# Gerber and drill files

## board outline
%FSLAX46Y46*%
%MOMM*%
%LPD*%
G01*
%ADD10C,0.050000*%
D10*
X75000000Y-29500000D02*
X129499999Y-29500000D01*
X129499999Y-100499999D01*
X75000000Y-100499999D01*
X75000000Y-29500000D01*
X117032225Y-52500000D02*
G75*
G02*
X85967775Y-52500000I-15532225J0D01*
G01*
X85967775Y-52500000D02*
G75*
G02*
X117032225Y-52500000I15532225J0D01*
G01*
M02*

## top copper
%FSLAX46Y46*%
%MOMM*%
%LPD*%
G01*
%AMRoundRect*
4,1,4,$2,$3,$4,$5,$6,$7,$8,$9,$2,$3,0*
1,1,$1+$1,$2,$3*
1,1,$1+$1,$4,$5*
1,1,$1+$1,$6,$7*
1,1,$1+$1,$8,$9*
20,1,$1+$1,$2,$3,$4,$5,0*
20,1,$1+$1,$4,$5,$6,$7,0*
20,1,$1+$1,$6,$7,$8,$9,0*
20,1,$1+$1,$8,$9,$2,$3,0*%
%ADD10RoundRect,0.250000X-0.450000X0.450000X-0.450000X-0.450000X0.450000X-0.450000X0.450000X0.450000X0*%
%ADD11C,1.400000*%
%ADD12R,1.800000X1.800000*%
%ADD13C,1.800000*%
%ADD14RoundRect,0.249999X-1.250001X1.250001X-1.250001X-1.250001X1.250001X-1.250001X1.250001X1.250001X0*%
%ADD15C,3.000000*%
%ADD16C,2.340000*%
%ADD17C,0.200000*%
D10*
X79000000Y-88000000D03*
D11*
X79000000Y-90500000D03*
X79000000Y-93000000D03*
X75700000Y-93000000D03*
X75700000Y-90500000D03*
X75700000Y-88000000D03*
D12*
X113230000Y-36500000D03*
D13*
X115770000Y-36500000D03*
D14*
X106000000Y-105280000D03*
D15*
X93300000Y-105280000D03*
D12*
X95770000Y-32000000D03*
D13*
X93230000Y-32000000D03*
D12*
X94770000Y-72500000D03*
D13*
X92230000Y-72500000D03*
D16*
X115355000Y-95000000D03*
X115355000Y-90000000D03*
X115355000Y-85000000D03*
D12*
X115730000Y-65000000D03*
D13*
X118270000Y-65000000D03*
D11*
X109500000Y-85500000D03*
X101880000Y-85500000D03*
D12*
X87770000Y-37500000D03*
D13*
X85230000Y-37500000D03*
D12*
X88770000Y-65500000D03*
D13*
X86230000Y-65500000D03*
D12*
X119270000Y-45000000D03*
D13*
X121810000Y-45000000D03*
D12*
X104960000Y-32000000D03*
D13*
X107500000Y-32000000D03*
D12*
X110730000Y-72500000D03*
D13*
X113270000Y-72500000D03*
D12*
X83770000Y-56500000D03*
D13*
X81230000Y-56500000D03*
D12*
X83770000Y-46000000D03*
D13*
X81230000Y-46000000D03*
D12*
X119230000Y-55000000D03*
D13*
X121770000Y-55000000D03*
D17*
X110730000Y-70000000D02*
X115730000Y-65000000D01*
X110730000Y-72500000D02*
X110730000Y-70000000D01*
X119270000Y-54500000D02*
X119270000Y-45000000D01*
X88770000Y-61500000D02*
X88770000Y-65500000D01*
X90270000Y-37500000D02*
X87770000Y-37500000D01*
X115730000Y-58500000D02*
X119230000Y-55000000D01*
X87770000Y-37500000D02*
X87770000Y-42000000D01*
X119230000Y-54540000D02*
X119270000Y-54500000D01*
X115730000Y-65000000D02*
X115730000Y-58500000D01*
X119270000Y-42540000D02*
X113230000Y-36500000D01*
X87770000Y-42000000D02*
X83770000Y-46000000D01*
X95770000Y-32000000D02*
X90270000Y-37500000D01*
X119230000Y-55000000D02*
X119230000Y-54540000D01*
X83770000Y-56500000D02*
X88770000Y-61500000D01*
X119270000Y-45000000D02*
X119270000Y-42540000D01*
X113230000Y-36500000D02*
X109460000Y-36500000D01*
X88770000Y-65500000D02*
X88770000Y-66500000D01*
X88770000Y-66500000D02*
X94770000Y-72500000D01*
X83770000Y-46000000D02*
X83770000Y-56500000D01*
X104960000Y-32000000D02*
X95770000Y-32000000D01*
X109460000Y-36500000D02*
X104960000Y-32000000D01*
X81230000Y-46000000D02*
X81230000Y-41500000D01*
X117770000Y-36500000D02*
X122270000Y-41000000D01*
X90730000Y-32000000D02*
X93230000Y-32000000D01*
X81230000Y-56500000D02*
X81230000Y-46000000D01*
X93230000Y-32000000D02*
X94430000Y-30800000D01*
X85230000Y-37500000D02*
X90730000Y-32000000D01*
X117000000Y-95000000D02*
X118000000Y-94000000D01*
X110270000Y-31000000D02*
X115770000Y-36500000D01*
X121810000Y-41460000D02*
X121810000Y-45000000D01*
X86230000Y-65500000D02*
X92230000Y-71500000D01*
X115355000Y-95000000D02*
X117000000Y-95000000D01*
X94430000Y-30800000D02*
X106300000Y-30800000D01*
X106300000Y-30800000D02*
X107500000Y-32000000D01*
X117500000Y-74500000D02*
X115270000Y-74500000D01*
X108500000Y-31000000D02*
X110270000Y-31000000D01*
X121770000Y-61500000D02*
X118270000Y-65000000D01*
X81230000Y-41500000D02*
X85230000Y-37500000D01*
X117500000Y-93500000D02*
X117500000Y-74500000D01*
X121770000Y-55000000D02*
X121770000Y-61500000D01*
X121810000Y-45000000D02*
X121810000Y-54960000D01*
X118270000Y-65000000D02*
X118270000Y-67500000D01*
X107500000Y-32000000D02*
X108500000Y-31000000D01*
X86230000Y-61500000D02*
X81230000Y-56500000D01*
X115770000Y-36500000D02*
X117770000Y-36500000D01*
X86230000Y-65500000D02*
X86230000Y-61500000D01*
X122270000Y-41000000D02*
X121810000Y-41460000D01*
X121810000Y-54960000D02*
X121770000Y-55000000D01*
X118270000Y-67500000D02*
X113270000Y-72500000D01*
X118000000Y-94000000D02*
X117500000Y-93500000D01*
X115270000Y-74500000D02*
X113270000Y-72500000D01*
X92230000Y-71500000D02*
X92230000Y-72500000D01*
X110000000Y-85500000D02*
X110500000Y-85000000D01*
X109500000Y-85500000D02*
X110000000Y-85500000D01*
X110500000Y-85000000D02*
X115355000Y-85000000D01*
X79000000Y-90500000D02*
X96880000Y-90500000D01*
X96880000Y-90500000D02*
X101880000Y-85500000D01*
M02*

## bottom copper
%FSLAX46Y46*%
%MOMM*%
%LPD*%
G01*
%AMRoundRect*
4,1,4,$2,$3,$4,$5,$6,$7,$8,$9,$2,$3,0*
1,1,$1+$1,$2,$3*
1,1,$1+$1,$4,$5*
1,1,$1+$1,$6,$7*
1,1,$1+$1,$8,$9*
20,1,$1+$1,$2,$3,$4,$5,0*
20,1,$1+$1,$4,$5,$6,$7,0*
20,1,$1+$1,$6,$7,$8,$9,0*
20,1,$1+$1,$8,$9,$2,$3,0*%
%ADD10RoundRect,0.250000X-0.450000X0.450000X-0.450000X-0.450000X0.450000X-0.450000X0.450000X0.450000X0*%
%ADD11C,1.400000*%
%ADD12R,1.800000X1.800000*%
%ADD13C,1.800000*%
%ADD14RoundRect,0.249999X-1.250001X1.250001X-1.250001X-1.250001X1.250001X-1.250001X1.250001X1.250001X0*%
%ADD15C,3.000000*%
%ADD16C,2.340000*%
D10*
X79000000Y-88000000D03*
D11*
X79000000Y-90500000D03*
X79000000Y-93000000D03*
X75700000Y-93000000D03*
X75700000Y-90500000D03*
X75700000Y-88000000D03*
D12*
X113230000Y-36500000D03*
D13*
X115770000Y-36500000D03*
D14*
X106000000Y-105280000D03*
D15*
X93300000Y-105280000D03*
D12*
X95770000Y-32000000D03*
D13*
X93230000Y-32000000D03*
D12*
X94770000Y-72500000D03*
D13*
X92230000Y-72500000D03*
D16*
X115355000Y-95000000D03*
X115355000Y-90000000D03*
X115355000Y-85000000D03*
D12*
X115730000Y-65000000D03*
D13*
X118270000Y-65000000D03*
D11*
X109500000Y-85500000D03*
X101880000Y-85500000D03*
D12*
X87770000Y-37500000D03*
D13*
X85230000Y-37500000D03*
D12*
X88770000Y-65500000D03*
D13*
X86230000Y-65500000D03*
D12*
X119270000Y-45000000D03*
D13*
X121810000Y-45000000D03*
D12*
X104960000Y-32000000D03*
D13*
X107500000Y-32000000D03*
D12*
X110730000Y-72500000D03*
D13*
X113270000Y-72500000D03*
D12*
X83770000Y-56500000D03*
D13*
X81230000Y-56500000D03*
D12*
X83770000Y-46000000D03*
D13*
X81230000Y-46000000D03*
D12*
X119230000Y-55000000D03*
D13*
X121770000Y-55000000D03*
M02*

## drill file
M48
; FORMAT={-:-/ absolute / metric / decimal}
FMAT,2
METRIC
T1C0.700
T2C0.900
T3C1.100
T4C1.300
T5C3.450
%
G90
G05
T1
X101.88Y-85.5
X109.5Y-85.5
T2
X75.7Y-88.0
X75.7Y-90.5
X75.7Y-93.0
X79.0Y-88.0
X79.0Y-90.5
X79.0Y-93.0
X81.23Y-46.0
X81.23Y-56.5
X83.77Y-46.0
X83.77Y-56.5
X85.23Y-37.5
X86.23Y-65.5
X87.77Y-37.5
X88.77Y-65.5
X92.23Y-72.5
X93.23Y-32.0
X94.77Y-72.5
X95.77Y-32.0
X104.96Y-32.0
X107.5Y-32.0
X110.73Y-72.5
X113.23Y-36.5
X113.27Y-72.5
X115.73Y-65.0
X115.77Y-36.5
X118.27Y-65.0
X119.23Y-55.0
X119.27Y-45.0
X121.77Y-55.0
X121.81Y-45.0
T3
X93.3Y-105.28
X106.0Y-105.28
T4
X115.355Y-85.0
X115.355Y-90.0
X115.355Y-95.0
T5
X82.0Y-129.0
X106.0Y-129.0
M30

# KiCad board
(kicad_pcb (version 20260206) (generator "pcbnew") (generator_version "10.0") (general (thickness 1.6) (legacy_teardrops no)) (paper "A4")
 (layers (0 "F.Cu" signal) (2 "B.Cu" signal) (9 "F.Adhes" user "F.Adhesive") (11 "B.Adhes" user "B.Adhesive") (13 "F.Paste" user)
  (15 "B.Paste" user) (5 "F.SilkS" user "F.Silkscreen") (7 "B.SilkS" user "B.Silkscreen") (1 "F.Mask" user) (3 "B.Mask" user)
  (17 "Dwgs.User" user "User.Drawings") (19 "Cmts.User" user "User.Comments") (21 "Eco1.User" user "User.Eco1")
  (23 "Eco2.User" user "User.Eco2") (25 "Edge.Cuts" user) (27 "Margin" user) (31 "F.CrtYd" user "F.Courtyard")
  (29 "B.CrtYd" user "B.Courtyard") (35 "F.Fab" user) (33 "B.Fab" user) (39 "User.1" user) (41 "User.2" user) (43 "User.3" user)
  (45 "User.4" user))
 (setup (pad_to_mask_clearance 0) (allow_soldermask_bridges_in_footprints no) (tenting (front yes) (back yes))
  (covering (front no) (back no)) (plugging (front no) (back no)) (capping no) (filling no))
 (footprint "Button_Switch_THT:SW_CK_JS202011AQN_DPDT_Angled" (layer "F.Cu") (at 79 88 -90)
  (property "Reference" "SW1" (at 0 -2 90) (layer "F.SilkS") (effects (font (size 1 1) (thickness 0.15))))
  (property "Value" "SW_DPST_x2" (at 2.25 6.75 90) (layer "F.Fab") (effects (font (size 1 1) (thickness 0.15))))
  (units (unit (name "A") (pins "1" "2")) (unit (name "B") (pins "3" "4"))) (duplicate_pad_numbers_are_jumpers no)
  (pad "1" thru_hole roundrect (at 0 0 270) (size 1.4 1.4) (drill 0.9) (layers "*.Cu" "*.Mask") (remove_unused_layers no)
   (roundrect_rratio 0.1785714286) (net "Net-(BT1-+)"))
  (pad "2" thru_hole circle (at 2.5 0 270) (size 1.4 1.4) (drill 0.9) (layers "*.Cu" "*.Mask") (remove_unused_layers no)
   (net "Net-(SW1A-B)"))
  (pad "3" thru_hole circle (at 5 0 270) (size 1.4 1.4) (drill 0.9) (layers "*.Cu" "*.Mask") (remove_unused_layers no))
  (pad "4" thru_hole circle (at 5 3.3 270) (size 1.4 1.4) (drill 0.9) (layers "*.Cu" "*.Mask") (remove_unused_layers no))
  (pad "5" thru_hole circle (at 2.5 3.3 270) (size 1.4 1.4) (drill 0.9) (layers "*.Cu" "*.Mask") (remove_unused_layers no))
  (pad "6" thru_hole circle (at 0 3.3 270) (size 1.4 1.4) (drill 0.9) (layers "*.Cu" "*.Mask") (remove_unused_layers no)))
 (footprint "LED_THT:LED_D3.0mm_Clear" (layer "F.Cu") (at 113.23 36.5)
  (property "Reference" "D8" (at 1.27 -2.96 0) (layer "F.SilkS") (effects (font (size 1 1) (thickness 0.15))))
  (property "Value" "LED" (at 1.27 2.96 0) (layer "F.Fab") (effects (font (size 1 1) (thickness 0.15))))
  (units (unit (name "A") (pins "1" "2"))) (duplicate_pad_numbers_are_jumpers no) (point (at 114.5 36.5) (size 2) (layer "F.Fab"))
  (pad "1" thru_hole rect (at 0 0) (size 1.8 1.8) (drill 0.9) (layers "*.Cu" "*.Mask") (remove_unused_layers no) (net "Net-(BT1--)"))
  (pad "2" thru_hole circle (at 2.54 0) (size 1.8 1.8) (drill 0.9) (layers "*.Cu" "*.Mask") (remove_unused_layers no) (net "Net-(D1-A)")))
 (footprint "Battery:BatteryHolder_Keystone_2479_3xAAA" (layer "F.Cu") (at 106 105.28 -90)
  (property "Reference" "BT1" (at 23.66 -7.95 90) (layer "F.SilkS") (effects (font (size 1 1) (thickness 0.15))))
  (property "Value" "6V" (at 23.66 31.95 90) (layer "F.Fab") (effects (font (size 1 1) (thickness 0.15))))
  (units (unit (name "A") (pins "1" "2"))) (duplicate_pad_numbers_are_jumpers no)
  (pad "" np_thru_hole circle (at 23.72 0 270) (size 3.45 3.45) (drill 3.45) (layers "*.Cu" "*.Mask"))
  (pad "" np_thru_hole circle (at 23.72 24 270) (size 3.45 3.45) (drill 3.45) (layers "*.Cu" "*.Mask"))
  (pad "1" thru_hole roundrect (at 0 0 270) (size 3 3) (drill 1.1) (layers "*.Cu" "*.Mask") (remove_unused_layers no)
   (roundrect_rratio 0.083333) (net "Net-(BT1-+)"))
  (pad "2" thru_hole circle (at 0 12.7 270) (size 3 3) (drill 1.1) (layers "*.Cu" "*.Mask") (remove_unused_layers no) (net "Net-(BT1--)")))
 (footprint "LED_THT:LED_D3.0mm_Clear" (layer "F.Cu") (at 95.77 32 180)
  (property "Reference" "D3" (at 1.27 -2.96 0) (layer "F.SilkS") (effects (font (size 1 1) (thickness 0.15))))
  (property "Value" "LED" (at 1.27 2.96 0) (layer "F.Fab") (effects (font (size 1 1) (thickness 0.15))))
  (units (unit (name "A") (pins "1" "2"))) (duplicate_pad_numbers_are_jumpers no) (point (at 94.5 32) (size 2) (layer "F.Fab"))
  (pad "1" thru_hole rect (at 0 0 180) (size 1.8 1.8) (drill 0.9) (layers "*.Cu" "*.Mask") (remove_unused_layers no) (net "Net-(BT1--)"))
  (pad "2" thru_hole circle (at 2.54 0 180) (size 1.8 1.8) (drill 0.9) (layers "*.Cu" "*.Mask") (remove_unused_layers no) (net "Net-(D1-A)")))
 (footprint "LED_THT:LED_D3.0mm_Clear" (layer "F.Cu") (at 94.77 72.5 180)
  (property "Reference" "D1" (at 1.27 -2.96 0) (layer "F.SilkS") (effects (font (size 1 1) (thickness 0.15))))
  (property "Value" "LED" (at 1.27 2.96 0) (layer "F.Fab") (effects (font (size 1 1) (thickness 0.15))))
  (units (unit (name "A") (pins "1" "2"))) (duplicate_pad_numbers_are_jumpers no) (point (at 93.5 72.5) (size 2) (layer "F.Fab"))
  (pad "1" thru_hole rect (at 0 0 180) (size 1.8 1.8) (drill 0.9) (layers "*.Cu" "*.Mask") (remove_unused_layers no) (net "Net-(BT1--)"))
  (pad "2" thru_hole circle (at 2.54 0 180) (size 1.8 1.8) (drill 0.9) (layers "*.Cu" "*.Mask") (remove_unused_layers no) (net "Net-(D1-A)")))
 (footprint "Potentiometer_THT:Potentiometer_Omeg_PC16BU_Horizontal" (layer "F.Cu") (at 115.355 95)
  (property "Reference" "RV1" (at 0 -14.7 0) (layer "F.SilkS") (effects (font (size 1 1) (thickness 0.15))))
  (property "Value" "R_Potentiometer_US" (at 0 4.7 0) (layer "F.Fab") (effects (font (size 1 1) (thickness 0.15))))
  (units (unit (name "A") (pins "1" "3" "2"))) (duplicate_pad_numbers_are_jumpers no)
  (pad "1" thru_hole circle (at 0 0) (size 2.34 2.34) (drill 1.3) (layers "*.Cu" "*.Mask") (remove_unused_layers no) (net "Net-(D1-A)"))
  (pad "2" thru_hole circle (at 0 -5) (size 2.34 2.34) (drill 1.3) (layers "*.Cu" "*.Mask") (remove_unused_layers no)
   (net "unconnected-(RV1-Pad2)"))
  (pad "3" thru_hole circle (at 0 -10) (size 2.34 2.34) (drill 1.3) (layers "*.Cu" "*.Mask") (remove_unused_layers no) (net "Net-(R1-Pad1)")))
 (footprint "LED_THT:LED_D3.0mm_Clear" (layer "F.Cu") (at 115.73 65)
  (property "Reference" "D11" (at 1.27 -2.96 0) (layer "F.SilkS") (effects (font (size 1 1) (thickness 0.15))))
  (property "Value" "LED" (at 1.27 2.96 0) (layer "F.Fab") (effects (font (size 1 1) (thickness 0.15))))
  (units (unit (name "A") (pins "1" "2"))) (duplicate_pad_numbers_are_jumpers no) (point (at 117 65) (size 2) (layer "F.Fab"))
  (pad "1" thru_hole rect (at 0 0) (size 1.8 1.8) (drill 0.9) (layers "*.Cu" "*.Mask") (remove_unused_layers no) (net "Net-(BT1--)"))
  (pad "2" thru_hole circle (at 2.54 0) (size 1.8 1.8) (drill 0.9) (layers "*.Cu" "*.Mask") (remove_unused_layers no) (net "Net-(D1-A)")))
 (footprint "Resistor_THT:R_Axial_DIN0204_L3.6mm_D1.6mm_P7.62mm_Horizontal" (layer "F.Cu") (at 109.5 85.5 180)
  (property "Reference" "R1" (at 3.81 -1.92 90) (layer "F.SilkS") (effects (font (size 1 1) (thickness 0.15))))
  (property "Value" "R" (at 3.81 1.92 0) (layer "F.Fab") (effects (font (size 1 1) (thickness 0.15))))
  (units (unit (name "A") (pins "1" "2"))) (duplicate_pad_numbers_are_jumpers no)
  (pad "1" thru_hole circle (at 0 0 180) (size 1.4 1.4) (drill 0.7) (layers "*.Cu" "*.Mask") (remove_unused_layers no) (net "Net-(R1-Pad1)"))
  (pad "2" thru_hole circle (at 7.62 0 180) (size 1.4 1.4) (drill 0.7) (layers "*.Cu" "*.Mask") (remove_unused_layers no)
   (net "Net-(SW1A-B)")))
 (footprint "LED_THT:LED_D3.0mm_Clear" (layer "F.Cu") (at 87.77 37.5 180)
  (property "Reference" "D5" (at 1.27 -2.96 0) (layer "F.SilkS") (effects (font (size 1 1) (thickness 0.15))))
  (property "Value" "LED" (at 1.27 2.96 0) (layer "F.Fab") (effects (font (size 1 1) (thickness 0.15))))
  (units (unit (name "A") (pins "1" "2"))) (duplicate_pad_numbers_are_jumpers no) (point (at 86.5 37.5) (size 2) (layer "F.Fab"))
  (pad "1" thru_hole rect (at 0 0 180) (size 1.8 1.8) (drill 0.9) (layers "*.Cu" "*.Mask") (remove_unused_layers no) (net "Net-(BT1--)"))
  (pad "2" thru_hole circle (at 2.54 0 180) (size 1.8 1.8) (drill 0.9) (layers "*.Cu" "*.Mask") (remove_unused_layers no) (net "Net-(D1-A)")))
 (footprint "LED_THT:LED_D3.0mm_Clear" (layer "F.Cu") (at 88.77 65.5 180)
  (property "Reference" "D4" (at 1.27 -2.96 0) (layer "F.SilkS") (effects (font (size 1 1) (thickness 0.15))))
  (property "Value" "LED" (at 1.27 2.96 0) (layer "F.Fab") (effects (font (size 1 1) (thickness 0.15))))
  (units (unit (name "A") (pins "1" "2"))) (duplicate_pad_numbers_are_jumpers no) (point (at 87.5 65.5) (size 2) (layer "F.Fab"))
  (pad "1" thru_hole rect (at 0 0 180) (size 1.8 1.8) (drill 0.9) (layers "*.Cu" "*.Mask") (remove_unused_layers no) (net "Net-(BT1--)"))
  (pad "2" thru_hole circle (at 2.54 0 180) (size 1.8 1.8) (drill 0.9) (layers "*.Cu" "*.Mask") (remove_unused_layers no) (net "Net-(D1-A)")))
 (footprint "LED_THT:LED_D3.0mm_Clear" (layer "F.Cu") (at 119.27 45)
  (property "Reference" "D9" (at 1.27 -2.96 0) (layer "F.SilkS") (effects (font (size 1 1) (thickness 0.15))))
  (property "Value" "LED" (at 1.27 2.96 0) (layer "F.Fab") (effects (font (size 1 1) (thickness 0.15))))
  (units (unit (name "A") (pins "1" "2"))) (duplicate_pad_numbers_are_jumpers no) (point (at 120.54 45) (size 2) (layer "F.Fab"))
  (pad "1" thru_hole rect (at 0 0) (size 1.8 1.8) (drill 0.9) (layers "*.Cu" "*.Mask") (remove_unused_layers no) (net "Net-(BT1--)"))
  (pad "2" thru_hole circle (at 2.54 0) (size 1.8 1.8) (drill 0.9) (layers "*.Cu" "*.Mask") (remove_unused_layers no) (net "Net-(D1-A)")))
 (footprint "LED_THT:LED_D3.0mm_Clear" (layer "F.Cu") (at 104.96 32)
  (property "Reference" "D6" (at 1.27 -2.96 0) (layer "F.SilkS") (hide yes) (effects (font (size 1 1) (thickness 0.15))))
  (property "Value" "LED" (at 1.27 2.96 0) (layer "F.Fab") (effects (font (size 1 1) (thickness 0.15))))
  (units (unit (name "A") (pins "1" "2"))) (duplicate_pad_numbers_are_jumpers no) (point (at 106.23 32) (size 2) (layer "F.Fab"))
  (pad "1" thru_hole rect (at 0 0) (size 1.8 1.8) (drill 0.9) (layers "*.Cu" "*.Mask") (remove_unused_layers no) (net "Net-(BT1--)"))
  (pad "2" thru_hole circle (at 2.54 0) (size 1.8 1.8) (drill 0.9) (layers "*.Cu" "*.Mask") (remove_unused_layers no) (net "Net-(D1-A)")))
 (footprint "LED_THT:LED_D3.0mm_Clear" (layer "F.Cu") (at 110.73 72.5)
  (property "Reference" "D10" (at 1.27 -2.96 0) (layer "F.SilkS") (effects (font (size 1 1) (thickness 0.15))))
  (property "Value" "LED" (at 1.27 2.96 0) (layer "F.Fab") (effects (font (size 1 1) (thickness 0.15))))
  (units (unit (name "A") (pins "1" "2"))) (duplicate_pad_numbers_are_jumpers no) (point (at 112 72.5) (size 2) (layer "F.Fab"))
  (pad "1" thru_hole rect (at 0 0) (size 1.8 1.8) (drill 0.9) (layers "*.Cu" "*.Mask") (remove_unused_layers no) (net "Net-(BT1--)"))
  (pad "2" thru_hole circle (at 2.54 0) (size 1.8 1.8) (drill 0.9) (layers "*.Cu" "*.Mask") (remove_unused_layers no) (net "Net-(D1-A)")))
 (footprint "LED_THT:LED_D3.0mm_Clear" (layer "F.Cu") (at 83.77 56.5 180)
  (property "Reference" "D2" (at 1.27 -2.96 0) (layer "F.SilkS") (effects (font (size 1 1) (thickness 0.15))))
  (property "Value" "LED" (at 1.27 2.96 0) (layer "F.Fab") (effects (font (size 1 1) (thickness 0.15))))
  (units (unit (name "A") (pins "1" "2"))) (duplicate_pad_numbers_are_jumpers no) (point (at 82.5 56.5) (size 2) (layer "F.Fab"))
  (pad "1" thru_hole rect (at 0 0 180) (size 1.8 1.8) (drill 0.9) (layers "*.Cu" "*.Mask") (remove_unused_layers no) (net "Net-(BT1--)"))
  (pad "2" thru_hole circle (at 2.54 0 180) (size 1.8 1.8) (drill 0.9) (layers "*.Cu" "*.Mask") (remove_unused_layers no) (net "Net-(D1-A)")))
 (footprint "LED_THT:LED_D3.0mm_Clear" (layer "F.Cu") (at 83.77 46 180)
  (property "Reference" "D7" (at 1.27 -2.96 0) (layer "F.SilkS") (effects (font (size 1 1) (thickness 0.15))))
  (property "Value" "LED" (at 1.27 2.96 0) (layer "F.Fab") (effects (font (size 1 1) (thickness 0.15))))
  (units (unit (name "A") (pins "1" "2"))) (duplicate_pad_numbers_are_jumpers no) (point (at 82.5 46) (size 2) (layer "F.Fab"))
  (pad "1" thru_hole rect (at 0 0 180) (size 1.8 1.8) (drill 0.9) (layers "*.Cu" "*.Mask") (remove_unused_layers no) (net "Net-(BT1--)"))
  (pad "2" thru_hole circle (at 2.54 0 180) (size 1.8 1.8) (drill 0.9) (layers "*.Cu" "*.Mask") (remove_unused_layers no) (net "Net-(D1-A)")))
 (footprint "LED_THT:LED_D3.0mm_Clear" (layer "F.Cu") (at 119.23 55)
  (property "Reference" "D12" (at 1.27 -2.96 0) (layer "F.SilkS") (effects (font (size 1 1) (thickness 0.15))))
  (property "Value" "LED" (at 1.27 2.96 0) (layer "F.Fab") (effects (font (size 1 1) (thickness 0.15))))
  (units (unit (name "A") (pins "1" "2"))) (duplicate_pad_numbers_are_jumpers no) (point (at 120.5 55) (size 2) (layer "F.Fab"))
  (pad "1" thru_hole rect (at 0 0) (size 1.8 1.8) (drill 0.9) (layers "*.Cu" "*.Mask") (remove_unused_layers no) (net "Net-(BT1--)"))
  (pad "2" thru_hole circle (at 2.54 0) (size 1.8 1.8) (drill 0.9) (layers "*.Cu" "*.Mask") (remove_unused_layers no) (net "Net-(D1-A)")))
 (gr_rect (start 75 29.5) (end 129.499999 100.499999) (stroke (width 0.05) (type default)) (fill no) (layer "Edge.Cuts"))
 (gr_circle (center 101.5 52.5) (end 102.5 68) (stroke (width 0.05) (type default)) (fill no) (layer "Edge.Cuts"))
 (segment (start 110.73 70) (end 115.73 65) (width 0.2) (layer "F.Cu") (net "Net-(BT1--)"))
 (segment (start 110.73 72.5) (end 110.73 70) (width 0.2) (layer "F.Cu") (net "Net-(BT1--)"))
 (segment (start 119.27 54.5) (end 119.27 45) (width 0.2) (layer "F.Cu") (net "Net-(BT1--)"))
 (segment (start 88.77 61.5) (end 88.77 65.5) (width 0.2) (layer "F.Cu") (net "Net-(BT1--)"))
 (segment (start 90.27 37.5) (end 87.77 37.5) (width 0.2) (layer "F.Cu") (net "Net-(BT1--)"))
 (segment (start 115.73 58.5) (end 119.23 55) (width 0.2) (layer "F.Cu") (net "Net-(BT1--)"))
 (segment (start 87.77 37.5) (end 87.77 42) (width 0.2) (layer "F.Cu") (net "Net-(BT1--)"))
 (segment (start 119.23 54.54) (end 119.27 54.5) (width 0.2) (layer "F.Cu") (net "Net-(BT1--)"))
 (segment (start 115.73 65) (end 115.73 58.5) (width 0.2) (layer "F.Cu") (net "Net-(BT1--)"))
 (segment (start 119.27 42.54) (end 113.23 36.5) (width 0.2) (layer "F.Cu") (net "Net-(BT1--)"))
 (segment (start 87.77 42) (end 83.77 46) (width 0.2) (layer "F.Cu") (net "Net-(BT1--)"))
 (segment (start 95.77 32) (end 90.27 37.5) (width 0.2) (layer "F.Cu") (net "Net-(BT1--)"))
 (segment (start 119.23 55) (end 119.23 54.54) (width 0.2) (layer "F.Cu") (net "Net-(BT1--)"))
 (segment (start 83.77 56.5) (end 88.77 61.5) (width 0.2) (layer "F.Cu") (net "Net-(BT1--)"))
 (segment (start 119.27 45) (end 119.27 42.54) (width 0.2) (layer "F.Cu") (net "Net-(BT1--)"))
 (segment (start 113.23 36.5) (end 109.46 36.5) (width 0.2) (layer "F.Cu") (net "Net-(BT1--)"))
 (segment (start 88.77 65.5) (end 88.77 66.5) (width 0.2) (layer "F.Cu") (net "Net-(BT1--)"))
 (segment (start 88.77 66.5) (end 94.77 72.5) (width 0.2) (layer "F.Cu") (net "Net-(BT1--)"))
 (segment (start 83.77 46) (end 83.77 56.5) (width 0.2) (layer "F.Cu") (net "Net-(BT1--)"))
 (segment (start 104.96 32) (end 95.77 32) (width 0.2) (layer "F.Cu") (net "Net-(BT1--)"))
 (segment (start 109.46 36.5) (end 104.96 32) (width 0.2) (layer "F.Cu") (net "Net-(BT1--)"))
 (segment (start 81.23 46) (end 81.23 41.5) (width 0.2) (layer "F.Cu") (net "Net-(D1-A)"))
 (segment (start 117.77 36.5) (end 122.27 41) (width 0.2) (layer "F.Cu") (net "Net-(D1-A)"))
 (segment (start 90.73 32) (end 93.23 32) (width 0.2) (layer "F.Cu") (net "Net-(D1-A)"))
 (segment (start 81.23 56.5) (end 81.23 46) (width 0.2) (layer "F.Cu") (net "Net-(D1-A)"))
 (segment (start 93.23 32) (end 94.43 30.8) (width 0.2) (layer "F.Cu") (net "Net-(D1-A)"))
 (segment (start 85.23 37.5) (end 90.73 32) (width 0.2) (layer "F.Cu") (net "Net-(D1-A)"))
 (segment (start 117 95) (end 118 94) (width 0.2) (layer "F.Cu") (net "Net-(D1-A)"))
 (segment (start 110.27 31) (end 115.77 36.5) (width 0.2) (layer "F.Cu") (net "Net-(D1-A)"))
 (segment (start 121.81 41.46) (end 121.81 45) (width 0.2) (layer "F.Cu") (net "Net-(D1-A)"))
 (segment (start 86.23 65.5) (end 92.23 71.5) (width 0.2) (layer "F.Cu") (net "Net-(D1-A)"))
 (segment (start 115.355 95) (end 117 95) (width 0.2) (layer "F.Cu") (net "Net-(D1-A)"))
 (segment (start 94.43 30.8) (end 106.3 30.8) (width 0.2) (layer "F.Cu") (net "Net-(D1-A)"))
 (segment (start 106.3 30.8) (end 107.5 32) (width 0.2) (layer "F.Cu") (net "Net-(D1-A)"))
 (segment (start 117.5 74.5) (end 115.27 74.5) (width 0.2) (layer "F.Cu") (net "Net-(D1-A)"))
 (segment (start 108.5 31) (end 110.27 31) (width 0.2) (layer "F.Cu") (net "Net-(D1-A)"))
 (segment (start 121.77 61.5) (end 118.27 65) (width 0.2) (layer "F.Cu") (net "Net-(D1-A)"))
 (segment (start 81.23 41.5) (end 85.23 37.5) (width 0.2) (layer "F.Cu") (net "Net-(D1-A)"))
 (segment (start 117.5 93.5) (end 117.5 74.5) (width 0.2) (layer "F.Cu") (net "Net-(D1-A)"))
 (segment (start 121.77 55) (end 121.77 61.5) (width 0.2) (layer "F.Cu") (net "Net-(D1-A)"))
 (segment (start 121.81 45) (end 121.81 54.96) (width 0.2) (layer "F.Cu") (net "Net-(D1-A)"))
 (segment (start 118.27 65) (end 118.27 67.5) (width 0.2) (layer "F.Cu") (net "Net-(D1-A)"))
 (segment (start 107.5 32) (end 108.5 31) (width 0.2) (layer "F.Cu") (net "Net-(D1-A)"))
 (segment (start 86.23 61.5) (end 81.23 56.5) (width 0.2) (layer "F.Cu") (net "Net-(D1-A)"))
 (segment (start 115.77 36.5) (end 117.77 36.5) (width 0.2) (layer "F.Cu") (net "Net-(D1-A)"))
 (segment (start 86.23 65.5) (end 86.23 61.5) (width 0.2) (layer "F.Cu") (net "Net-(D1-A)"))
 (segment (start 122.27 41) (end 121.81 41.46) (width 0.2) (layer "F.Cu") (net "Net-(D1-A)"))
 (segment (start 121.81 54.96) (end 121.77 55) (width 0.2) (layer "F.Cu") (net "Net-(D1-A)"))
 (segment (start 118.27 67.5) (end 113.27 72.5) (width 0.2) (layer "F.Cu") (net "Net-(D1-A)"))
 (segment (start 118 94) (end 117.5 93.5) (width 0.2) (layer "F.Cu") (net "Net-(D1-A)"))
 (segment (start 115.27 74.5) (end 113.27 72.5) (width 0.2) (layer "F.Cu") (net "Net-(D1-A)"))
 (segment (start 92.23 71.5) (end 92.23 72.5) (width 0.2) (layer "F.Cu") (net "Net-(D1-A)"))
 (segment (start 110 85.5) (end 110.5 85) (width 0.2) (layer "F.Cu") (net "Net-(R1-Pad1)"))
 (segment (start 109.5 85.5) (end 110 85.5) (width 0.2) (layer "F.Cu") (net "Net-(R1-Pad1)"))
 (segment (start 110.5 85) (end 115.355 85) (width 0.2) (layer "F.Cu") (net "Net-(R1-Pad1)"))
 (segment (start 79 90.5) (end 96.88 90.5) (width 0.2) (layer "F.Cu") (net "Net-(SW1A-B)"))
 (segment (start 96.88 90.5) (end 101.88 85.5) (width 0.2) (layer "F.Cu") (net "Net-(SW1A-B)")))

